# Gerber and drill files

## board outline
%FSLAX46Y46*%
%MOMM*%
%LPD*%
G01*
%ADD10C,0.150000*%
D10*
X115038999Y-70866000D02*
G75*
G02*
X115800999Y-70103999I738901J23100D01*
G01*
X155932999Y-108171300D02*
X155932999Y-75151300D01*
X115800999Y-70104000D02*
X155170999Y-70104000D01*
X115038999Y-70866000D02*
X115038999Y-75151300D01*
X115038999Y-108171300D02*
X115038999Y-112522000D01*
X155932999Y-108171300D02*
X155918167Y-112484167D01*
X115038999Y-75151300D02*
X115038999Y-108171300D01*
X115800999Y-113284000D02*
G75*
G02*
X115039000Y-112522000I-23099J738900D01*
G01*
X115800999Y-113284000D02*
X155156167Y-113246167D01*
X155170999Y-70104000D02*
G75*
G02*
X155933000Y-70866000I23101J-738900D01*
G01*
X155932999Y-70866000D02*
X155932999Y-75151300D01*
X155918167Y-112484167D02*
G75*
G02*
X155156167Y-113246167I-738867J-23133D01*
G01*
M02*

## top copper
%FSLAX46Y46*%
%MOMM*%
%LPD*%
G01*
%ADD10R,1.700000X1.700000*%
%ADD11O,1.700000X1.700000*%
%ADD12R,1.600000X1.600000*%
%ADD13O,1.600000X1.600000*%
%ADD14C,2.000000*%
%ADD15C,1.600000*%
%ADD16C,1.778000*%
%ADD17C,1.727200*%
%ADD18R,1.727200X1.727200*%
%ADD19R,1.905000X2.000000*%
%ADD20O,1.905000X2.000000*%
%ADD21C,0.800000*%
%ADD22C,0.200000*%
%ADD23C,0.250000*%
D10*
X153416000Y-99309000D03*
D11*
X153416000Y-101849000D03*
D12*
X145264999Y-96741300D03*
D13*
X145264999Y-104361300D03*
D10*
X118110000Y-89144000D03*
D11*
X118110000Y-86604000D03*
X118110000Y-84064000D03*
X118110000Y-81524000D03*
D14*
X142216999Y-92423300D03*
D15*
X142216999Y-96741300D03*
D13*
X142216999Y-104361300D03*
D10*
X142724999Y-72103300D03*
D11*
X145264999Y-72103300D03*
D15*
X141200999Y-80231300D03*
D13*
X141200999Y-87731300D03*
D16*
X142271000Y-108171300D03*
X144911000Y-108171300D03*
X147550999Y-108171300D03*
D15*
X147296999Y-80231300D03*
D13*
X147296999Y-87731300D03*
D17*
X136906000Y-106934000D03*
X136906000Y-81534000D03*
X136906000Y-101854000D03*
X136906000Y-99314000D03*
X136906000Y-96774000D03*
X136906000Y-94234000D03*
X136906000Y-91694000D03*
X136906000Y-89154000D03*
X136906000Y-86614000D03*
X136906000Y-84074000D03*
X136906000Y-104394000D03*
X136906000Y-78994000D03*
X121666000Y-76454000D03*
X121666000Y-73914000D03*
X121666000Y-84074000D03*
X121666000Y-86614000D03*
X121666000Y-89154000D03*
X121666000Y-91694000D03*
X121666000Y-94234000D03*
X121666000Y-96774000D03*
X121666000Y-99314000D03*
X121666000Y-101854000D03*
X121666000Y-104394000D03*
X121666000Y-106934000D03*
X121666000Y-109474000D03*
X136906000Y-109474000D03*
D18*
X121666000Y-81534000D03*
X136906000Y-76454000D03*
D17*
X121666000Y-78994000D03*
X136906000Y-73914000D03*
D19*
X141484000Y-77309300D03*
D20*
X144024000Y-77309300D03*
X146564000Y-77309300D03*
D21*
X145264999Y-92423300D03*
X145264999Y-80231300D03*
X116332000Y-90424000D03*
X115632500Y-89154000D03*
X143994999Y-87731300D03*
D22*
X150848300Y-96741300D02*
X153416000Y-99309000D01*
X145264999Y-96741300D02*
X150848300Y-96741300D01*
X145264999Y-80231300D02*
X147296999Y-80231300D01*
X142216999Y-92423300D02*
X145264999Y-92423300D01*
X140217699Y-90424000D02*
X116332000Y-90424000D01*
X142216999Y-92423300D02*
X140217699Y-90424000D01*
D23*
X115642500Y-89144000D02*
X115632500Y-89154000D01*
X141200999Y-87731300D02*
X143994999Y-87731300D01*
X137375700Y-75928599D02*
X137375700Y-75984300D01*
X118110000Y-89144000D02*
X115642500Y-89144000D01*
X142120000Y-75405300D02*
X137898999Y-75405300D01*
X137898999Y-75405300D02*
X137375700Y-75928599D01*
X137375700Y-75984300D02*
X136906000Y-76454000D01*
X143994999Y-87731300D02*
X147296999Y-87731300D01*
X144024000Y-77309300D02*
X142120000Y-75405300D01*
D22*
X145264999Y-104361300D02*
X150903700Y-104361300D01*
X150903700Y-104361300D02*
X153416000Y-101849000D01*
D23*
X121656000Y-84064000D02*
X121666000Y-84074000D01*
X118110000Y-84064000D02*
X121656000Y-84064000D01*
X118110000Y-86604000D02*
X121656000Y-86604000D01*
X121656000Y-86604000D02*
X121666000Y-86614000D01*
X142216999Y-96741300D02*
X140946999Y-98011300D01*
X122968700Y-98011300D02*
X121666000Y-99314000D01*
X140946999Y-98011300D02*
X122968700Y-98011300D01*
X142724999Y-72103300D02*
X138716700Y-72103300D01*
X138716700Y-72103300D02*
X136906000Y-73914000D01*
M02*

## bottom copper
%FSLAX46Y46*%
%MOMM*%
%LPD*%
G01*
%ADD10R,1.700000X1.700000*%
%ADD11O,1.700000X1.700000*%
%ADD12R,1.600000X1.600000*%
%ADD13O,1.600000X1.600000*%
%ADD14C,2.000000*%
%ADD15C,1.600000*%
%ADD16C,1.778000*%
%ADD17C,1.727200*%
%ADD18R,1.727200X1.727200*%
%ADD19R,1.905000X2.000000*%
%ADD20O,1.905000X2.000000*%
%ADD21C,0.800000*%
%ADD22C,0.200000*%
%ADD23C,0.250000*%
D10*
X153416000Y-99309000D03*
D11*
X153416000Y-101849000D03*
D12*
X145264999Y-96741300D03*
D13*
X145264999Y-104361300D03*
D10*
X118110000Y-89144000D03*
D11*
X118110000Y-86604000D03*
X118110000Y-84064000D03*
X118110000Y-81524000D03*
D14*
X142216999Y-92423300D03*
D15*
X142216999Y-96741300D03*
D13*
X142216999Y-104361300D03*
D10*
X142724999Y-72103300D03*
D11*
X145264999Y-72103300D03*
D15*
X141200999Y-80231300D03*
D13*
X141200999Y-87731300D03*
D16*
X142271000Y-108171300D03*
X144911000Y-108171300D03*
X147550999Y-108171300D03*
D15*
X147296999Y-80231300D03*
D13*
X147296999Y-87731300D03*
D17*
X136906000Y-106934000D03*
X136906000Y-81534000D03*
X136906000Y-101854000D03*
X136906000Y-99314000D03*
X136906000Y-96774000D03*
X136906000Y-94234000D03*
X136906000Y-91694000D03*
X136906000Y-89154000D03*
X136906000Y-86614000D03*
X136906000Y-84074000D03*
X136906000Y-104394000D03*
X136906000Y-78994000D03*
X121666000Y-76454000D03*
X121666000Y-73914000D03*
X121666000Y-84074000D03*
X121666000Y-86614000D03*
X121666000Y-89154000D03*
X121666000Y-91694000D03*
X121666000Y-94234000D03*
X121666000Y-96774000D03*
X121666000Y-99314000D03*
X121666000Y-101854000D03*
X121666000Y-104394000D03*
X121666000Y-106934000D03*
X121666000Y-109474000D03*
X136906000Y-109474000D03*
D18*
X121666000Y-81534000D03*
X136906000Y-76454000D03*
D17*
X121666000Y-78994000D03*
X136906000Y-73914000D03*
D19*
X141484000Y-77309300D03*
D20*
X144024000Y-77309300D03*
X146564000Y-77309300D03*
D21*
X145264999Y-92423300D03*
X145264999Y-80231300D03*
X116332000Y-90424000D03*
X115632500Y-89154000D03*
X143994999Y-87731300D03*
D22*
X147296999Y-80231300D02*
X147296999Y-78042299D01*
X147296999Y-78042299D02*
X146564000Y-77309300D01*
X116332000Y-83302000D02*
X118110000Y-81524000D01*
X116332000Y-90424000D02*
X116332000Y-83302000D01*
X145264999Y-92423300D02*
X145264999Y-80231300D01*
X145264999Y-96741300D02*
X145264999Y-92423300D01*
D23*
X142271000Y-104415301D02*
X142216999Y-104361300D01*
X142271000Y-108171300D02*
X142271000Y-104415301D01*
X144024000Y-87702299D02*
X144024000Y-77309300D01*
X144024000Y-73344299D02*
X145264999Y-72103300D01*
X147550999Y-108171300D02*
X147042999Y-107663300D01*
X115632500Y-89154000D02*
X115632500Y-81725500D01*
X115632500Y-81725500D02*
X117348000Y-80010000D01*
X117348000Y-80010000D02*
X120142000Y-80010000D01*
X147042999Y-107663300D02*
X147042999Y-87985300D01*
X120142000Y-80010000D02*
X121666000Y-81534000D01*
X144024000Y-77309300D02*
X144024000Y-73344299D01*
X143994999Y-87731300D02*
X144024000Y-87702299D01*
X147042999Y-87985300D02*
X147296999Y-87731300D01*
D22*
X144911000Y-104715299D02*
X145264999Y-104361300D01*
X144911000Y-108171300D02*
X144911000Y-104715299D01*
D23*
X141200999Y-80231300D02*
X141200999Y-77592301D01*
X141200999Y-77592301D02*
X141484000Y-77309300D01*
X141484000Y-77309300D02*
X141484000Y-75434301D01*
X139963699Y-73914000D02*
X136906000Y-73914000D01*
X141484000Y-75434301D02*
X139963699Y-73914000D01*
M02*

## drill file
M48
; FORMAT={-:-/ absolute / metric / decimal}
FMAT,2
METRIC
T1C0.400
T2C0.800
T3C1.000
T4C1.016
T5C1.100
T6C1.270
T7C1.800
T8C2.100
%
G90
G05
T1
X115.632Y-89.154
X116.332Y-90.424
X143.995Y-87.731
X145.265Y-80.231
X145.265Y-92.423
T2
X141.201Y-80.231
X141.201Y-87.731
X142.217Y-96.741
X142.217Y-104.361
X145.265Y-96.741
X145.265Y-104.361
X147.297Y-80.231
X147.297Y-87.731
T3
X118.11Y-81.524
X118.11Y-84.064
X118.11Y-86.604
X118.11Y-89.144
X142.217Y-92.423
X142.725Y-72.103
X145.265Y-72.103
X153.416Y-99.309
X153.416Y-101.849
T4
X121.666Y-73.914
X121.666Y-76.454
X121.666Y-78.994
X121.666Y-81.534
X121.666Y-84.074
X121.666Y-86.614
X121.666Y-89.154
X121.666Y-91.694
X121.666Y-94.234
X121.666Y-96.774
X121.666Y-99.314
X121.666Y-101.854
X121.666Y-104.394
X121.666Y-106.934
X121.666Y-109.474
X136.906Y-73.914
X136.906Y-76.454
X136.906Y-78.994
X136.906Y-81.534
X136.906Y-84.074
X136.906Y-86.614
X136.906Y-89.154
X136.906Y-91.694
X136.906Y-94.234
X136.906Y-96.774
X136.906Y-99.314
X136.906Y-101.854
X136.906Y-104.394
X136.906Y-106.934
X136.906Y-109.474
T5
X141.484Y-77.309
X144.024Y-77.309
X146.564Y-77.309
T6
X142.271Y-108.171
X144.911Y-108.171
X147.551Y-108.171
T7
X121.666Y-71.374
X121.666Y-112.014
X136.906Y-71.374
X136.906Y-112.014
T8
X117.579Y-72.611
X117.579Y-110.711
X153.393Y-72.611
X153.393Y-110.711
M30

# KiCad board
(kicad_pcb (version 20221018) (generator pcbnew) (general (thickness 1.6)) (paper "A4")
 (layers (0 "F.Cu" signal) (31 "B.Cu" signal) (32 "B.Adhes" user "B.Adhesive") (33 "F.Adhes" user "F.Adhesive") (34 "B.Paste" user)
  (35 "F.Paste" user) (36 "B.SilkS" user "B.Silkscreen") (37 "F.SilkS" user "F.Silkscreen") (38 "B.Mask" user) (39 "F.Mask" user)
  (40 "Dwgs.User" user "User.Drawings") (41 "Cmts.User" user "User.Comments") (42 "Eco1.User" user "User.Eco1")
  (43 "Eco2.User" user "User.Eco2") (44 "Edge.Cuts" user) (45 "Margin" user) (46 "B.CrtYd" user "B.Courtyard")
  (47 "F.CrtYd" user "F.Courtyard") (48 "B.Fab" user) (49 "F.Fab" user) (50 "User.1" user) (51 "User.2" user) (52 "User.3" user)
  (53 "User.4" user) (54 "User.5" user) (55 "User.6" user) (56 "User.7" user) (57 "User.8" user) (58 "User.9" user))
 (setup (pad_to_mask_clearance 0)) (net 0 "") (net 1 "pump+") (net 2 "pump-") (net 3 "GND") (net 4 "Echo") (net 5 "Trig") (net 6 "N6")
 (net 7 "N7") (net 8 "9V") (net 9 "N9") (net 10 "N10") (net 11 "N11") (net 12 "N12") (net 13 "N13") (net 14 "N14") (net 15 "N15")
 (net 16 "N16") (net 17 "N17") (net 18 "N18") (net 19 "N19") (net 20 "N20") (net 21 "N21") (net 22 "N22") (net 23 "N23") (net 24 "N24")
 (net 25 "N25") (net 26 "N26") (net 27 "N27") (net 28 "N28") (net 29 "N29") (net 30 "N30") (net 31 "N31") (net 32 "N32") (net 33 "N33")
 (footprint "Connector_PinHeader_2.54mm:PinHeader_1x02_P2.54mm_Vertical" (layer "F.Cu") (at 153.416 99.309)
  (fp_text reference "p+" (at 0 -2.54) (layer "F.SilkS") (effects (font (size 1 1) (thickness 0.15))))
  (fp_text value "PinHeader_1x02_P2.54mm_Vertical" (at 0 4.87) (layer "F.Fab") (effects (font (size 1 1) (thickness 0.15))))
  (pad "1" thru_hole rect (at 0 0) (size 1.7 1.7) (drill 1) (layers "*.Cu" "*.Mask") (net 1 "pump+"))
  (pad "2" thru_hole oval (at 0 2.54) (size 1.7 1.7) (drill 1) (layers "*.Cu" "*.Mask") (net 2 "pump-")))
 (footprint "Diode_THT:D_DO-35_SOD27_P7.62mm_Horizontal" (layer "F.Cu") (at 145.264999 96.7413 -90)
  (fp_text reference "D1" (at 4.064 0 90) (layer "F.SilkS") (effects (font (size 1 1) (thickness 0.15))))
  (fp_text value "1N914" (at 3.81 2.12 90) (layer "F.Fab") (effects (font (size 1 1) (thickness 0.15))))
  (pad "1" thru_hole rect (at 0 0 270) (size 1.6 1.6) (drill 0.8) (layers "*.Cu" "*.Mask") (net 1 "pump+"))
  (pad "2" thru_hole oval (at 7.62 0 270) (size 1.6 1.6) (drill 0.8) (layers "*.Cu" "*.Mask") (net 2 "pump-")))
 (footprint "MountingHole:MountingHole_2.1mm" (layer "F.Cu") (at 153.392999 72.6113)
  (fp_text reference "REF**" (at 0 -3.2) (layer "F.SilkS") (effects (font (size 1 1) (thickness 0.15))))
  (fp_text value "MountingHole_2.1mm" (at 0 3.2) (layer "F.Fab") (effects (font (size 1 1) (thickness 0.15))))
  (pad "" np_thru_hole circle (at 0 0) (size 2.1 2.1) (drill 2.1) (layers "F&B.Cu" "*.Mask")))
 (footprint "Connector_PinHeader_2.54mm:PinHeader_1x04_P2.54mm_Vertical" (layer "F.Cu") (at 118.11 89.144 180)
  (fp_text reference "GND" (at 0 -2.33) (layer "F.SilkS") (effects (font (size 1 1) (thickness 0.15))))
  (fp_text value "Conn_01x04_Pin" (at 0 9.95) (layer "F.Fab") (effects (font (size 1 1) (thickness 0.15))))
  (pad "1" thru_hole rect (at 0 0 180) (size 1.7 1.7) (drill 1) (layers "*.Cu" "*.Mask") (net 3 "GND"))
  (pad "2" thru_hole oval (at 0 2.54 180) (size 1.7 1.7) (drill 1) (layers "*.Cu" "*.Mask") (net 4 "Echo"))
  (pad "3" thru_hole oval (at 0 5.08 180) (size 1.7 1.7) (drill 1) (layers "*.Cu" "*.Mask") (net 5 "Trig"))
  (pad "4" thru_hole oval (at 0 7.62 180) (size 1.7 1.7) (drill 1) (layers "*.Cu" "*.Mask") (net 1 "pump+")))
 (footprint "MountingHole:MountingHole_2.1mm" (layer "F.Cu") (at 117.578999 72.6113)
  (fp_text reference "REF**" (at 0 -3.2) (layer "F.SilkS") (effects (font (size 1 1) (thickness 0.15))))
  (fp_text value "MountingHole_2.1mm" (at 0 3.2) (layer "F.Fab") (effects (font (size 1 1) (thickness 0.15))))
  (pad "" np_thru_hole circle (at 0 0) (size 2.1 2.1) (drill 2.1) (layers "*.Cu" "*.Mask")))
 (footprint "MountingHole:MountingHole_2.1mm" (layer "F.Cu") (at 153.392999 110.7113)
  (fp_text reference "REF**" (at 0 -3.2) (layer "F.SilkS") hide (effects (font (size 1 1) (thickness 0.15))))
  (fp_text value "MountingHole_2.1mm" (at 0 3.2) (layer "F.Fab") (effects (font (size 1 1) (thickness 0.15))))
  (pad "" np_thru_hole circle (at 0 0) (size 2.1 2.1) (drill 2.1) (layers "F&B.Cu" "*.Mask")))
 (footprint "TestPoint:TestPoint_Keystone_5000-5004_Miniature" (layer "F.Cu") (at 142.216999 92.4233)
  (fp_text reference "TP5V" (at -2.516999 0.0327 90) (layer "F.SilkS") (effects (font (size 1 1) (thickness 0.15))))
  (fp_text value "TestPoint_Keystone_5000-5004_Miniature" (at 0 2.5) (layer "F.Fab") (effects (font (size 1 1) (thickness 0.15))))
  (pad "1" thru_hole circle (at 0 0) (size 2 2) (drill 1) (layers "*.Cu" "*.Mask") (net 1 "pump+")))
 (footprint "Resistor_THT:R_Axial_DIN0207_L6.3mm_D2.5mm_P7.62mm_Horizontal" (layer "F.Cu") (at 142.216999 96.7413 -90)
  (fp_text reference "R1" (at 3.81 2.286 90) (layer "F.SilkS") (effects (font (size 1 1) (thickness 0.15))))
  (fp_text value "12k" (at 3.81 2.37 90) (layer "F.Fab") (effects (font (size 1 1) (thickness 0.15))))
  (pad "1" thru_hole circle (at 0 0 270) (size 1.6 1.6) (drill 0.8) (layers "*.Cu" "*.Mask") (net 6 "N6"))
  (pad "2" thru_hole oval (at 7.62 0 270) (size 1.6 1.6) (drill 0.8) (layers "*.Cu" "*.Mask") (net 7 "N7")))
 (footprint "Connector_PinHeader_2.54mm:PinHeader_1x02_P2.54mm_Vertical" (layer "F.Cu") (at 142.724999 72.1033 90)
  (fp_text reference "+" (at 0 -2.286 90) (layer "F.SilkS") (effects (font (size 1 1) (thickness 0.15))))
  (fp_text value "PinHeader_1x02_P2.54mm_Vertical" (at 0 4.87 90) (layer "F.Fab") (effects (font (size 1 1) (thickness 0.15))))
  (pad "1" thru_hole rect (at 0 0 90) (size 1.7 1.7) (drill 1) (layers "*.Cu" "*.Mask") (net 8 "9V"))
  (pad "2" thru_hole oval (at 0 2.54 90) (size 1.7 1.7) (drill 1) (layers "*.Cu" "*.Mask") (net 3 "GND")))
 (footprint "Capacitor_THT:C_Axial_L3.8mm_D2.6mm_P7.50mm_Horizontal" (layer "F.Cu") (at 141.200999 80.2313 -90)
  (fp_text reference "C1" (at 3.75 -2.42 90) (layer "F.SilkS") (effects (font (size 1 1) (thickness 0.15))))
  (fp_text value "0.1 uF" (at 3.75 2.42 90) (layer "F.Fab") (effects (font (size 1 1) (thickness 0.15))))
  (pad "1" thru_hole circle (at 0 0 270) (size 1.6 1.6) (drill 0.8) (layers "*.Cu" "*.Mask") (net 8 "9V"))
  (pad "2" thru_hole oval (at 7.5 0 270) (size 1.6 1.6) (drill 0.8) (layers "*.Cu" "*.Mask") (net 3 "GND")))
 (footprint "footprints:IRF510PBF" (layer "F.Cu") (at 142.271 108.1713)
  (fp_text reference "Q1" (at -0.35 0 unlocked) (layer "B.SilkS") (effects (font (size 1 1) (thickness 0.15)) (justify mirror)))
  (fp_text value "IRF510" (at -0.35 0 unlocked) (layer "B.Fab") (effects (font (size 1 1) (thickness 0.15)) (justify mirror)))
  (pad "1" thru_hole circle (at 0 0) (size 1.778 1.778) (drill 1.27) (layers "*.Cu" "*.Mask") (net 7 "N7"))
  (pad "2" thru_hole circle (at 2.64 0) (size 1.778 1.778) (drill 1.27) (layers "*.Cu" "*.Mask") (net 2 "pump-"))
  (pad "3" thru_hole circle (at 5.279999 0) (size 1.778 1.778) (drill 1.27) (layers "*.Cu" "*.Mask") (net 3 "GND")))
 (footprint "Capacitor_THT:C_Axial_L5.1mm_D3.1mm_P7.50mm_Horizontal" (layer "F.Cu") (at 147.296999 80.2313 -90)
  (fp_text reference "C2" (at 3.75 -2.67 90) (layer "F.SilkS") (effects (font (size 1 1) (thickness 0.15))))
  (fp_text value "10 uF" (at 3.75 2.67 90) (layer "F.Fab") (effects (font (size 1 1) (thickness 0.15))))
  (pad "1" thru_hole circle (at 0 0 270) (size 1.6 1.6) (drill 0.8) (layers "*.Cu" "*.Mask") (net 1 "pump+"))
  (pad "2" thru_hole oval (at 7.5 0 270) (size 1.6 1.6) (drill 0.8) (layers "*.Cu" "*.Mask") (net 3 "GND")))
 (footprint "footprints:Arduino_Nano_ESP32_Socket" (layer "F.Cu") (at 129.286 113.284)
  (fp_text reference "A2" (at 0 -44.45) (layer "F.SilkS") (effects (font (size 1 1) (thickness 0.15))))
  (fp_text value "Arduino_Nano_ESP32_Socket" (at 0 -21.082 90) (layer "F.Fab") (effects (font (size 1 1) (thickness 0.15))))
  (pad "" np_thru_hole circle (at -7.62 -41.91) (size 1.8 1.8) (drill 1.8) (layers "F&B.Cu" "*.Mask"))
  (pad "" np_thru_hole circle (at -7.62 -1.27) (size 1.8 1.8) (drill 1.8) (layers "F&B.Cu" "*.Mask"))
  (pad "" np_thru_hole circle (at 7.62 -41.91) (size 1.8 1.8) (drill 1.8) (layers "F&B.Cu" "*.Mask"))
  (pad "" np_thru_hole circle (at 7.62 -1.27) (size 1.8 1.8) (drill 1.8) (layers "F&B.Cu" "*.Mask"))
  (pad "3V3" thru_hole circle (at 7.62 -6.35) (size 1.7272 1.7272) (drill 1.016) (layers "*.Cu" "*.Mask") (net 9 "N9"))
  (pad "5V" thru_hole circle (at 7.62 -31.75) (size 1.7272 1.7272) (drill 1.016) (layers "*.Cu" "*.Mask") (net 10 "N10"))
  (pad "A0" thru_hole circle (at 7.62 -11.43) (size 1.7272 1.7272) (drill 1.016) (layers "*.Cu" "*.Mask") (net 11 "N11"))
  (pad "A1" thru_hole circle (at 7.62 -13.97) (size 1.7272 1.7272) (drill 1.016) (layers "*.Cu" "*.Mask") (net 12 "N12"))
  (pad "A2" thru_hole circle (at 7.62 -16.51) (size 1.7272 1.7272) (drill 1.016) (layers "*.Cu" "*.Mask") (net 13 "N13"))
  (pad "A3" thru_hole circle (at 7.62 -19.05) (size 1.7272 1.7272) (drill 1.016) (layers "*.Cu" "*.Mask") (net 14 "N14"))
  (pad "A4" thru_hole circle (at 7.62 -21.59) (size 1.7272 1.7272) (drill 1.016) (layers "*.Cu" "*.Mask") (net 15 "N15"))
  (pad "A5" thru_hole circle (at 7.62 -24.13) (size 1.7272 1.7272) (drill 1.016) (layers "*.Cu" "*.Mask") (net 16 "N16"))
  (pad "A6" thru_hole circle (at 7.62 -26.67) (size 1.7272 1.7272) (drill 1.016) (layers "*.Cu" "*.Mask") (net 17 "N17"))
  (pad "A7" thru_hole circle (at 7.62 -29.21) (size 1.7272 1.7272) (drill 1.016) (layers "*.Cu" "*.Mask") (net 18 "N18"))
  (pad "B0" thru_hole circle (at 7.62 -8.89) (size 1.7272 1.7272) (drill 1.016) (layers "*.Cu" "*.Mask") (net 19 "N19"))
  (pad "B1" thru_hole circle (at 7.62 -34.29) (size 1.7272 1.7272) (drill 1.016) (layers "*.Cu" "*.Mask") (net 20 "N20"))
  (pad "D0" thru_hole circle (at -7.62 -36.83) (size 1.7272 1.7272) (drill 1.016) (layers "*.Cu" "*.Mask") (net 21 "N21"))
  (pad "D1" thru_hole circle (at -7.62 -39.37) (size 1.7272 1.7272) (drill 1.016) (layers "*.Cu" "*.Mask") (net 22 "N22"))
  (pad "D2" thru_hole circle (at -7.62 -29.21) (size 1.7272 1.7272) (drill 1.016) (layers "*.Cu" "*.Mask") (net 5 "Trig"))
  (pad "D3" thru_hole circle (at -7.62 -26.67) (size 1.7272 1.7272) (drill 1.016) (layers "*.Cu" "*.Mask") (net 4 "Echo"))
  (pad "D4" thru_hole circle (at -7.62 -24.13) (size 1.7272 1.7272) (drill 1.016) (layers "*.Cu" "*.Mask") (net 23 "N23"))
  (pad "D5" thru_hole circle (at -7.62 -21.59) (size 1.7272 1.7272) (drill 1.016) (layers "*.Cu" "*.Mask") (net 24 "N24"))
  (pad "D6" thru_hole circle (at -7.62 -19.05) (size 1.7272 1.7272) (drill 1.016) (layers "*.Cu" "*.Mask") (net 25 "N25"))
  (pad "D7" thru_hole circle (at -7.62 -16.51) (size 1.7272 1.7272) (drill 1.016) (layers "*.Cu" "*.Mask") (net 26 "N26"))
  (pad "D8" thru_hole circle (at -7.62 -13.97) (size 1.7272 1.7272) (drill 1.016) (layers "*.Cu" "*.Mask") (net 6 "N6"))
  (pad "D9" thru_hole circle (at -7.62 -11.43) (size 1.7272 1.7272) (drill 1.016) (layers "*.Cu" "*.Mask") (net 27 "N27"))
  (pad "D10" thru_hole circle (at -7.62 -8.89) (size 1.7272 1.7272) (drill 1.016) (layers "*.Cu" "*.Mask") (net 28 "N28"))
  (pad "D11" thru_hole circle (at -7.62 -6.35) (size 1.7272 1.7272) (drill 1.016) (layers "*.Cu" "*.Mask") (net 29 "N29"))
  (pad "D12" thru_hole circle (at -7.62 -3.81) (size 1.7272 1.7272) (drill 1.016) (layers "*.Cu" "*.Mask") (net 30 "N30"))
  (pad "D13" thru_hole circle (at 7.62 -3.81) (size 1.7272 1.7272) (drill 1.016) (layers "*.Cu" "*.Mask") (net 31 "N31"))
  (pad "GND1" thru_hole rect (at -7.62 -31.75) (size 1.7272 1.7272) (drill 1.016) (layers "*.Cu" "*.Mask") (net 3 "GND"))
  (pad "GND2" thru_hole rect (at 7.62 -36.83) (size 1.7272 1.7272) (drill 1.016) (layers "*.Cu" "*.Mask") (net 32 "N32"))
  (pad "RST" thru_hole circle (at -7.62 -34.29) (size 1.7272 1.7272) (drill 1.016) (layers "*.Cu" "*.Mask") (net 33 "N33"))
  (pad "VIN" thru_hole circle (at 7.62 -39.37) (size 1.7272 1.7272) (drill 1.016) (layers "*.Cu" "*.Mask") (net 8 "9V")))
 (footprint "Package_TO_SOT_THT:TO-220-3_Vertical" (layer "F.Cu") (at 141.484 77.3093)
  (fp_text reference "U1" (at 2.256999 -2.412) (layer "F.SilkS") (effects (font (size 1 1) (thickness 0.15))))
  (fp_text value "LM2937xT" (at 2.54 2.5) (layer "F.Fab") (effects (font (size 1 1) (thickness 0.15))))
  (pad "1" thru_hole rect (at 0 0) (size 1.905 2) (drill 1.1) (layers "*.Cu" "*.Mask") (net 8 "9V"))
  (pad "2" thru_hole oval (at 2.54 0) (size 1.905 2) (drill 1.1) (layers "*.Cu" "*.Mask") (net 3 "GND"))
  (pad "3" thru_hole oval (at 5.08 0) (size 1.905 2) (drill 1.1) (layers "*.Cu" "*.Mask") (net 1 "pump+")))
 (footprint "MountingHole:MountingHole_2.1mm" (layer "F.Cu") (at 117.578999 110.7113)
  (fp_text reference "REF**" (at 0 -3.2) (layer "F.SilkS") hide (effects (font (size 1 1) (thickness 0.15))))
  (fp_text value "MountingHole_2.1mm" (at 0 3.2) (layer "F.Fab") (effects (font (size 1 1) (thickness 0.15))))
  (pad "" np_thru_hole circle (at 0 0) (size 2.1 2.1) (drill 2.1) (layers "F&B.Cu" "*.Mask")))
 (gr_arc (start 115.038999 70.866) (mid 115.255166 70.320167) (end 115.800999 70.104) (stroke (width 0.15) (type default))
  (layer "Edge.Cuts"))
 (gr_line (start 155.932999 108.1713) (end 155.932999 75.1513) (stroke (width 0.15) (type default)) (layer "Edge.Cuts"))
 (gr_line (start 115.800999 70.104) (end 155.170999 70.104) (stroke (width 0.15) (type default)) (layer "Edge.Cuts"))
 (gr_line (start 115.038999 70.866) (end 115.038999 75.1513) (stroke (width 0.15) (type default)) (layer "Edge.Cuts"))
 (gr_line (start 115.038999 108.1713) (end 115.038999 112.522) (stroke (width 0.15) (type default)) (layer "Edge.Cuts"))
 (gr_line (start 155.932999 108.1713) (end 155.918167 112.484167) (stroke (width 0.15) (type default)) (layer "Edge.Cuts"))
 (gr_line (start 115.038999 75.1513) (end 115.038999 108.1713) (stroke (width 0.15) (type default)) (layer "Edge.Cuts"))
 (gr_arc (start 115.800999 113.284) (mid 115.255166 113.067833) (end 115.038999 112.522) (stroke (width 0.15) (type default))
  (layer "Edge.Cuts"))
 (gr_line (start 115.800999 113.284) (end 155.156167 113.246167) (stroke (width 0.15) (type default)) (layer "Edge.Cuts"))
 (gr_arc (start 155.170999 70.104) (mid 155.716832 70.320167) (end 155.932999 70.866) (stroke (width 0.15) (type default))
  (layer "Edge.Cuts"))
 (gr_line (start 155.932999 70.866) (end 155.932999 75.1513) (stroke (width 0.15) (type default)) (layer "Edge.Cuts"))
 (gr_arc (start 155.918167 112.484167) (mid 155.702 113.03) (end 155.156167 113.246167) (stroke (width 0.15) (type default))
  (layer "Edge.Cuts"))
 (segment (start 150.8483 96.7413) (end 153.416 99.309) (width 0.2) (layer "F.Cu") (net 1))
 (segment (start 145.264999 96.7413) (end 150.8483 96.7413) (width 0.2) (layer "F.Cu") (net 1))
 (segment (start 145.264999 80.2313) (end 147.296999 80.2313) (width 0.2) (layer "F.Cu") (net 1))
 (segment (start 142.216999 92.4233) (end 145.264999 92.4233) (width 0.2) (layer "F.Cu") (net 1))
 (segment (start 140.217699 90.424) (end 116.332 90.424) (width 0.2) (layer "F.Cu") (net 1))
 (segment (start 142.216999 92.4233) (end 140.217699 90.424) (width 0.2) (layer "F.Cu") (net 1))
 (via (at 145.264999 92.4233) (size 0.8) (drill 0.4) (layers "F.Cu" "B.Cu") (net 1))
 (via (at 145.264999 80.2313) (size 0.8) (drill 0.4) (layers "F.Cu" "B.Cu") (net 1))
 (via (at 116.332 90.424) (size 0.8) (drill 0.4) (layers "F.Cu" "B.Cu") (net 1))
 (segment (start 147.296999 80.2313) (end 147.296999 78.042299) (width 0.2) (layer "B.Cu") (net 1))
 (segment (start 147.296999 78.042299) (end 146.564 77.3093) (width 0.2) (layer "B.Cu") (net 1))
 (segment (start 116.332 83.302) (end 118.11 81.524) (width 0.2) (layer "B.Cu") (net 1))
 (segment (start 116.332 90.424) (end 116.332 83.302) (width 0.2) (layer "B.Cu") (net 1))
 (segment (start 145.264999 92.4233) (end 145.264999 80.2313) (width 0.2) (layer "B.Cu") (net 1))
 (segment (start 145.264999 96.7413) (end 145.264999 92.4233) (width 0.2) (layer "B.Cu") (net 1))
 (segment (start 142.271 104.415301) (end 142.216999 104.3613) (width 0.25) (layer "B.Cu") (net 7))
 (segment (start 142.271 108.1713) (end 142.271 104.415301) (width 0.25) (layer "B.Cu") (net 7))
 (segment (start 115.6425 89.144) (end 115.6325 89.154) (width 0.25) (layer "F.Cu") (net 3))
 (segment (start 141.200999 87.7313) (end 143.994999 87.7313) (width 0.25) (layer "F.Cu") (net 3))
 (segment (start 137.3757 75.928599) (end 137.3757 75.9843) (width 0.25) (layer "F.Cu") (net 3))
 (segment (start 118.11 89.144) (end 115.6425 89.144) (width 0.25) (layer "F.Cu") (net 3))
 (segment (start 142.12 75.4053) (end 137.898999 75.4053) (width 0.25) (layer "F.Cu") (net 3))
 (segment (start 137.898999 75.4053) (end 137.3757 75.928599) (width 0.25) (layer "F.Cu") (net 3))
 (segment (start 137.3757 75.9843) (end 136.906 76.454) (width 0.25) (layer "F.Cu") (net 3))
 (segment (start 143.994999 87.7313) (end 147.296999 87.7313) (width 0.25) (layer "F.Cu") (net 3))
 (segment (start 144.024 77.3093) (end 142.12 75.4053) (width 0.25) (layer "F.Cu") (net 3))
 (via (at 115.6325 89.154) (size 0.8) (drill 0.4) (layers "F.Cu" "B.Cu") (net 3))
 (via (at 143.994999 87.7313) (size 0.8) (drill 0.4) (layers "F.Cu" "B.Cu") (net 3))
 (segment (start 144.024 87.702299) (end 144.024 77.3093) (width 0.25) (layer "B.Cu") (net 3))
 (segment (start 144.024 73.344299) (end 145.264999 72.1033) (width 0.25) (layer "B.Cu") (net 3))
 (segment (start 147.550999 108.1713) (end 147.042999 107.6633) (width 0.25) (layer "B.Cu") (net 3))
 (segment (start 115.6325 89.154) (end 115.6325 81.7255) (width 0.25) (layer "B.Cu") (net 3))
 (segment (start 115.6325 81.7255) (end 117.348 80.01) (width 0.25) (layer "B.Cu") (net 3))
 (segment (start 117.348 80.01) (end 120.142 80.01) (width 0.25) (layer "B.Cu") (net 3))
 (segment (start 147.042999 107.6633) (end 147.042999 87.9853) (width 0.25) (layer "B.Cu") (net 3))
 (segment (start 120.142 80.01) (end 121.666 81.534) (width 0.25) (layer "B.Cu") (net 3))
 (segment (start 144.024 77.3093) (end 144.024 73.344299) (width 0.25) (layer "B.Cu") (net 3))
 (segment (start 143.994999 87.7313) (end 144.024 87.702299) (width 0.25) (layer "B.Cu") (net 3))
 (segment (start 147.042999 87.9853) (end 147.296999 87.7313) (width 0.25) (layer "B.Cu") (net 3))
 (segment (start 145.264999 104.3613) (end 150.9037 104.3613) (width 0.2) (layer "F.Cu") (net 2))
 (segment (start 150.9037 104.3613) (end 153.416 101.849) (width 0.2) (layer "F.Cu") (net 2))
 (segment (start 144.911 104.715299) (end 145.264999 104.3613) (width 0.2) (layer "B.Cu") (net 2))
 (segment (start 144.911 108.1713) (end 144.911 104.715299) (width 0.2) (layer "B.Cu") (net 2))
 (segment (start 121.656 84.064) (end 121.666 84.074) (width 0.25) (layer "F.Cu") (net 5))
 (segment (start 118.11 84.064) (end 121.656 84.064) (width 0.25) (layer "F.Cu") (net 5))
 (segment (start 118.11 86.604) (end 121.656 86.604) (width 0.25) (layer "F.Cu") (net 4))
 (segment (start 121.656 86.604) (end 121.666 86.614) (width 0.25) (layer "F.Cu") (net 4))
 (segment (start 142.216999 96.7413) (end 140.946999 98.0113) (width 0.25) (layer "F.Cu") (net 6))
 (segment (start 122.9687 98.0113) (end 121.666 99.314) (width 0.25) (layer "F.Cu") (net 6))
 (segment (start 140.946999 98.0113) (end 122.9687 98.0113) (width 0.25) (layer "F.Cu") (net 6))
 (segment (start 142.724999 72.1033) (end 138.7167 72.1033) (width 0.25) (layer "F.Cu") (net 8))
 (segment (start 138.7167 72.1033) (end 136.906 73.914) (width 0.25) (layer "F.Cu") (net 8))
 (segment (start 141.200999 80.2313) (end 141.200999 77.592301) (width 0.25) (layer "B.Cu") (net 8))
 (segment (start 141.200999 77.592301) (end 141.484 77.3093) (width 0.25) (layer "B.Cu") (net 8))
 (segment (start 141.484 77.3093) (end 141.484 75.434301) (width 0.25) (layer "B.Cu") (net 8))
 (segment (start 139.963699 73.914) (end 136.906 73.914) (width 0.25) (layer "B.Cu") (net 8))
 (segment (start 141.484 75.434301) (end 139.963699 73.914) (width 0.25) (layer "B.Cu") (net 8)))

